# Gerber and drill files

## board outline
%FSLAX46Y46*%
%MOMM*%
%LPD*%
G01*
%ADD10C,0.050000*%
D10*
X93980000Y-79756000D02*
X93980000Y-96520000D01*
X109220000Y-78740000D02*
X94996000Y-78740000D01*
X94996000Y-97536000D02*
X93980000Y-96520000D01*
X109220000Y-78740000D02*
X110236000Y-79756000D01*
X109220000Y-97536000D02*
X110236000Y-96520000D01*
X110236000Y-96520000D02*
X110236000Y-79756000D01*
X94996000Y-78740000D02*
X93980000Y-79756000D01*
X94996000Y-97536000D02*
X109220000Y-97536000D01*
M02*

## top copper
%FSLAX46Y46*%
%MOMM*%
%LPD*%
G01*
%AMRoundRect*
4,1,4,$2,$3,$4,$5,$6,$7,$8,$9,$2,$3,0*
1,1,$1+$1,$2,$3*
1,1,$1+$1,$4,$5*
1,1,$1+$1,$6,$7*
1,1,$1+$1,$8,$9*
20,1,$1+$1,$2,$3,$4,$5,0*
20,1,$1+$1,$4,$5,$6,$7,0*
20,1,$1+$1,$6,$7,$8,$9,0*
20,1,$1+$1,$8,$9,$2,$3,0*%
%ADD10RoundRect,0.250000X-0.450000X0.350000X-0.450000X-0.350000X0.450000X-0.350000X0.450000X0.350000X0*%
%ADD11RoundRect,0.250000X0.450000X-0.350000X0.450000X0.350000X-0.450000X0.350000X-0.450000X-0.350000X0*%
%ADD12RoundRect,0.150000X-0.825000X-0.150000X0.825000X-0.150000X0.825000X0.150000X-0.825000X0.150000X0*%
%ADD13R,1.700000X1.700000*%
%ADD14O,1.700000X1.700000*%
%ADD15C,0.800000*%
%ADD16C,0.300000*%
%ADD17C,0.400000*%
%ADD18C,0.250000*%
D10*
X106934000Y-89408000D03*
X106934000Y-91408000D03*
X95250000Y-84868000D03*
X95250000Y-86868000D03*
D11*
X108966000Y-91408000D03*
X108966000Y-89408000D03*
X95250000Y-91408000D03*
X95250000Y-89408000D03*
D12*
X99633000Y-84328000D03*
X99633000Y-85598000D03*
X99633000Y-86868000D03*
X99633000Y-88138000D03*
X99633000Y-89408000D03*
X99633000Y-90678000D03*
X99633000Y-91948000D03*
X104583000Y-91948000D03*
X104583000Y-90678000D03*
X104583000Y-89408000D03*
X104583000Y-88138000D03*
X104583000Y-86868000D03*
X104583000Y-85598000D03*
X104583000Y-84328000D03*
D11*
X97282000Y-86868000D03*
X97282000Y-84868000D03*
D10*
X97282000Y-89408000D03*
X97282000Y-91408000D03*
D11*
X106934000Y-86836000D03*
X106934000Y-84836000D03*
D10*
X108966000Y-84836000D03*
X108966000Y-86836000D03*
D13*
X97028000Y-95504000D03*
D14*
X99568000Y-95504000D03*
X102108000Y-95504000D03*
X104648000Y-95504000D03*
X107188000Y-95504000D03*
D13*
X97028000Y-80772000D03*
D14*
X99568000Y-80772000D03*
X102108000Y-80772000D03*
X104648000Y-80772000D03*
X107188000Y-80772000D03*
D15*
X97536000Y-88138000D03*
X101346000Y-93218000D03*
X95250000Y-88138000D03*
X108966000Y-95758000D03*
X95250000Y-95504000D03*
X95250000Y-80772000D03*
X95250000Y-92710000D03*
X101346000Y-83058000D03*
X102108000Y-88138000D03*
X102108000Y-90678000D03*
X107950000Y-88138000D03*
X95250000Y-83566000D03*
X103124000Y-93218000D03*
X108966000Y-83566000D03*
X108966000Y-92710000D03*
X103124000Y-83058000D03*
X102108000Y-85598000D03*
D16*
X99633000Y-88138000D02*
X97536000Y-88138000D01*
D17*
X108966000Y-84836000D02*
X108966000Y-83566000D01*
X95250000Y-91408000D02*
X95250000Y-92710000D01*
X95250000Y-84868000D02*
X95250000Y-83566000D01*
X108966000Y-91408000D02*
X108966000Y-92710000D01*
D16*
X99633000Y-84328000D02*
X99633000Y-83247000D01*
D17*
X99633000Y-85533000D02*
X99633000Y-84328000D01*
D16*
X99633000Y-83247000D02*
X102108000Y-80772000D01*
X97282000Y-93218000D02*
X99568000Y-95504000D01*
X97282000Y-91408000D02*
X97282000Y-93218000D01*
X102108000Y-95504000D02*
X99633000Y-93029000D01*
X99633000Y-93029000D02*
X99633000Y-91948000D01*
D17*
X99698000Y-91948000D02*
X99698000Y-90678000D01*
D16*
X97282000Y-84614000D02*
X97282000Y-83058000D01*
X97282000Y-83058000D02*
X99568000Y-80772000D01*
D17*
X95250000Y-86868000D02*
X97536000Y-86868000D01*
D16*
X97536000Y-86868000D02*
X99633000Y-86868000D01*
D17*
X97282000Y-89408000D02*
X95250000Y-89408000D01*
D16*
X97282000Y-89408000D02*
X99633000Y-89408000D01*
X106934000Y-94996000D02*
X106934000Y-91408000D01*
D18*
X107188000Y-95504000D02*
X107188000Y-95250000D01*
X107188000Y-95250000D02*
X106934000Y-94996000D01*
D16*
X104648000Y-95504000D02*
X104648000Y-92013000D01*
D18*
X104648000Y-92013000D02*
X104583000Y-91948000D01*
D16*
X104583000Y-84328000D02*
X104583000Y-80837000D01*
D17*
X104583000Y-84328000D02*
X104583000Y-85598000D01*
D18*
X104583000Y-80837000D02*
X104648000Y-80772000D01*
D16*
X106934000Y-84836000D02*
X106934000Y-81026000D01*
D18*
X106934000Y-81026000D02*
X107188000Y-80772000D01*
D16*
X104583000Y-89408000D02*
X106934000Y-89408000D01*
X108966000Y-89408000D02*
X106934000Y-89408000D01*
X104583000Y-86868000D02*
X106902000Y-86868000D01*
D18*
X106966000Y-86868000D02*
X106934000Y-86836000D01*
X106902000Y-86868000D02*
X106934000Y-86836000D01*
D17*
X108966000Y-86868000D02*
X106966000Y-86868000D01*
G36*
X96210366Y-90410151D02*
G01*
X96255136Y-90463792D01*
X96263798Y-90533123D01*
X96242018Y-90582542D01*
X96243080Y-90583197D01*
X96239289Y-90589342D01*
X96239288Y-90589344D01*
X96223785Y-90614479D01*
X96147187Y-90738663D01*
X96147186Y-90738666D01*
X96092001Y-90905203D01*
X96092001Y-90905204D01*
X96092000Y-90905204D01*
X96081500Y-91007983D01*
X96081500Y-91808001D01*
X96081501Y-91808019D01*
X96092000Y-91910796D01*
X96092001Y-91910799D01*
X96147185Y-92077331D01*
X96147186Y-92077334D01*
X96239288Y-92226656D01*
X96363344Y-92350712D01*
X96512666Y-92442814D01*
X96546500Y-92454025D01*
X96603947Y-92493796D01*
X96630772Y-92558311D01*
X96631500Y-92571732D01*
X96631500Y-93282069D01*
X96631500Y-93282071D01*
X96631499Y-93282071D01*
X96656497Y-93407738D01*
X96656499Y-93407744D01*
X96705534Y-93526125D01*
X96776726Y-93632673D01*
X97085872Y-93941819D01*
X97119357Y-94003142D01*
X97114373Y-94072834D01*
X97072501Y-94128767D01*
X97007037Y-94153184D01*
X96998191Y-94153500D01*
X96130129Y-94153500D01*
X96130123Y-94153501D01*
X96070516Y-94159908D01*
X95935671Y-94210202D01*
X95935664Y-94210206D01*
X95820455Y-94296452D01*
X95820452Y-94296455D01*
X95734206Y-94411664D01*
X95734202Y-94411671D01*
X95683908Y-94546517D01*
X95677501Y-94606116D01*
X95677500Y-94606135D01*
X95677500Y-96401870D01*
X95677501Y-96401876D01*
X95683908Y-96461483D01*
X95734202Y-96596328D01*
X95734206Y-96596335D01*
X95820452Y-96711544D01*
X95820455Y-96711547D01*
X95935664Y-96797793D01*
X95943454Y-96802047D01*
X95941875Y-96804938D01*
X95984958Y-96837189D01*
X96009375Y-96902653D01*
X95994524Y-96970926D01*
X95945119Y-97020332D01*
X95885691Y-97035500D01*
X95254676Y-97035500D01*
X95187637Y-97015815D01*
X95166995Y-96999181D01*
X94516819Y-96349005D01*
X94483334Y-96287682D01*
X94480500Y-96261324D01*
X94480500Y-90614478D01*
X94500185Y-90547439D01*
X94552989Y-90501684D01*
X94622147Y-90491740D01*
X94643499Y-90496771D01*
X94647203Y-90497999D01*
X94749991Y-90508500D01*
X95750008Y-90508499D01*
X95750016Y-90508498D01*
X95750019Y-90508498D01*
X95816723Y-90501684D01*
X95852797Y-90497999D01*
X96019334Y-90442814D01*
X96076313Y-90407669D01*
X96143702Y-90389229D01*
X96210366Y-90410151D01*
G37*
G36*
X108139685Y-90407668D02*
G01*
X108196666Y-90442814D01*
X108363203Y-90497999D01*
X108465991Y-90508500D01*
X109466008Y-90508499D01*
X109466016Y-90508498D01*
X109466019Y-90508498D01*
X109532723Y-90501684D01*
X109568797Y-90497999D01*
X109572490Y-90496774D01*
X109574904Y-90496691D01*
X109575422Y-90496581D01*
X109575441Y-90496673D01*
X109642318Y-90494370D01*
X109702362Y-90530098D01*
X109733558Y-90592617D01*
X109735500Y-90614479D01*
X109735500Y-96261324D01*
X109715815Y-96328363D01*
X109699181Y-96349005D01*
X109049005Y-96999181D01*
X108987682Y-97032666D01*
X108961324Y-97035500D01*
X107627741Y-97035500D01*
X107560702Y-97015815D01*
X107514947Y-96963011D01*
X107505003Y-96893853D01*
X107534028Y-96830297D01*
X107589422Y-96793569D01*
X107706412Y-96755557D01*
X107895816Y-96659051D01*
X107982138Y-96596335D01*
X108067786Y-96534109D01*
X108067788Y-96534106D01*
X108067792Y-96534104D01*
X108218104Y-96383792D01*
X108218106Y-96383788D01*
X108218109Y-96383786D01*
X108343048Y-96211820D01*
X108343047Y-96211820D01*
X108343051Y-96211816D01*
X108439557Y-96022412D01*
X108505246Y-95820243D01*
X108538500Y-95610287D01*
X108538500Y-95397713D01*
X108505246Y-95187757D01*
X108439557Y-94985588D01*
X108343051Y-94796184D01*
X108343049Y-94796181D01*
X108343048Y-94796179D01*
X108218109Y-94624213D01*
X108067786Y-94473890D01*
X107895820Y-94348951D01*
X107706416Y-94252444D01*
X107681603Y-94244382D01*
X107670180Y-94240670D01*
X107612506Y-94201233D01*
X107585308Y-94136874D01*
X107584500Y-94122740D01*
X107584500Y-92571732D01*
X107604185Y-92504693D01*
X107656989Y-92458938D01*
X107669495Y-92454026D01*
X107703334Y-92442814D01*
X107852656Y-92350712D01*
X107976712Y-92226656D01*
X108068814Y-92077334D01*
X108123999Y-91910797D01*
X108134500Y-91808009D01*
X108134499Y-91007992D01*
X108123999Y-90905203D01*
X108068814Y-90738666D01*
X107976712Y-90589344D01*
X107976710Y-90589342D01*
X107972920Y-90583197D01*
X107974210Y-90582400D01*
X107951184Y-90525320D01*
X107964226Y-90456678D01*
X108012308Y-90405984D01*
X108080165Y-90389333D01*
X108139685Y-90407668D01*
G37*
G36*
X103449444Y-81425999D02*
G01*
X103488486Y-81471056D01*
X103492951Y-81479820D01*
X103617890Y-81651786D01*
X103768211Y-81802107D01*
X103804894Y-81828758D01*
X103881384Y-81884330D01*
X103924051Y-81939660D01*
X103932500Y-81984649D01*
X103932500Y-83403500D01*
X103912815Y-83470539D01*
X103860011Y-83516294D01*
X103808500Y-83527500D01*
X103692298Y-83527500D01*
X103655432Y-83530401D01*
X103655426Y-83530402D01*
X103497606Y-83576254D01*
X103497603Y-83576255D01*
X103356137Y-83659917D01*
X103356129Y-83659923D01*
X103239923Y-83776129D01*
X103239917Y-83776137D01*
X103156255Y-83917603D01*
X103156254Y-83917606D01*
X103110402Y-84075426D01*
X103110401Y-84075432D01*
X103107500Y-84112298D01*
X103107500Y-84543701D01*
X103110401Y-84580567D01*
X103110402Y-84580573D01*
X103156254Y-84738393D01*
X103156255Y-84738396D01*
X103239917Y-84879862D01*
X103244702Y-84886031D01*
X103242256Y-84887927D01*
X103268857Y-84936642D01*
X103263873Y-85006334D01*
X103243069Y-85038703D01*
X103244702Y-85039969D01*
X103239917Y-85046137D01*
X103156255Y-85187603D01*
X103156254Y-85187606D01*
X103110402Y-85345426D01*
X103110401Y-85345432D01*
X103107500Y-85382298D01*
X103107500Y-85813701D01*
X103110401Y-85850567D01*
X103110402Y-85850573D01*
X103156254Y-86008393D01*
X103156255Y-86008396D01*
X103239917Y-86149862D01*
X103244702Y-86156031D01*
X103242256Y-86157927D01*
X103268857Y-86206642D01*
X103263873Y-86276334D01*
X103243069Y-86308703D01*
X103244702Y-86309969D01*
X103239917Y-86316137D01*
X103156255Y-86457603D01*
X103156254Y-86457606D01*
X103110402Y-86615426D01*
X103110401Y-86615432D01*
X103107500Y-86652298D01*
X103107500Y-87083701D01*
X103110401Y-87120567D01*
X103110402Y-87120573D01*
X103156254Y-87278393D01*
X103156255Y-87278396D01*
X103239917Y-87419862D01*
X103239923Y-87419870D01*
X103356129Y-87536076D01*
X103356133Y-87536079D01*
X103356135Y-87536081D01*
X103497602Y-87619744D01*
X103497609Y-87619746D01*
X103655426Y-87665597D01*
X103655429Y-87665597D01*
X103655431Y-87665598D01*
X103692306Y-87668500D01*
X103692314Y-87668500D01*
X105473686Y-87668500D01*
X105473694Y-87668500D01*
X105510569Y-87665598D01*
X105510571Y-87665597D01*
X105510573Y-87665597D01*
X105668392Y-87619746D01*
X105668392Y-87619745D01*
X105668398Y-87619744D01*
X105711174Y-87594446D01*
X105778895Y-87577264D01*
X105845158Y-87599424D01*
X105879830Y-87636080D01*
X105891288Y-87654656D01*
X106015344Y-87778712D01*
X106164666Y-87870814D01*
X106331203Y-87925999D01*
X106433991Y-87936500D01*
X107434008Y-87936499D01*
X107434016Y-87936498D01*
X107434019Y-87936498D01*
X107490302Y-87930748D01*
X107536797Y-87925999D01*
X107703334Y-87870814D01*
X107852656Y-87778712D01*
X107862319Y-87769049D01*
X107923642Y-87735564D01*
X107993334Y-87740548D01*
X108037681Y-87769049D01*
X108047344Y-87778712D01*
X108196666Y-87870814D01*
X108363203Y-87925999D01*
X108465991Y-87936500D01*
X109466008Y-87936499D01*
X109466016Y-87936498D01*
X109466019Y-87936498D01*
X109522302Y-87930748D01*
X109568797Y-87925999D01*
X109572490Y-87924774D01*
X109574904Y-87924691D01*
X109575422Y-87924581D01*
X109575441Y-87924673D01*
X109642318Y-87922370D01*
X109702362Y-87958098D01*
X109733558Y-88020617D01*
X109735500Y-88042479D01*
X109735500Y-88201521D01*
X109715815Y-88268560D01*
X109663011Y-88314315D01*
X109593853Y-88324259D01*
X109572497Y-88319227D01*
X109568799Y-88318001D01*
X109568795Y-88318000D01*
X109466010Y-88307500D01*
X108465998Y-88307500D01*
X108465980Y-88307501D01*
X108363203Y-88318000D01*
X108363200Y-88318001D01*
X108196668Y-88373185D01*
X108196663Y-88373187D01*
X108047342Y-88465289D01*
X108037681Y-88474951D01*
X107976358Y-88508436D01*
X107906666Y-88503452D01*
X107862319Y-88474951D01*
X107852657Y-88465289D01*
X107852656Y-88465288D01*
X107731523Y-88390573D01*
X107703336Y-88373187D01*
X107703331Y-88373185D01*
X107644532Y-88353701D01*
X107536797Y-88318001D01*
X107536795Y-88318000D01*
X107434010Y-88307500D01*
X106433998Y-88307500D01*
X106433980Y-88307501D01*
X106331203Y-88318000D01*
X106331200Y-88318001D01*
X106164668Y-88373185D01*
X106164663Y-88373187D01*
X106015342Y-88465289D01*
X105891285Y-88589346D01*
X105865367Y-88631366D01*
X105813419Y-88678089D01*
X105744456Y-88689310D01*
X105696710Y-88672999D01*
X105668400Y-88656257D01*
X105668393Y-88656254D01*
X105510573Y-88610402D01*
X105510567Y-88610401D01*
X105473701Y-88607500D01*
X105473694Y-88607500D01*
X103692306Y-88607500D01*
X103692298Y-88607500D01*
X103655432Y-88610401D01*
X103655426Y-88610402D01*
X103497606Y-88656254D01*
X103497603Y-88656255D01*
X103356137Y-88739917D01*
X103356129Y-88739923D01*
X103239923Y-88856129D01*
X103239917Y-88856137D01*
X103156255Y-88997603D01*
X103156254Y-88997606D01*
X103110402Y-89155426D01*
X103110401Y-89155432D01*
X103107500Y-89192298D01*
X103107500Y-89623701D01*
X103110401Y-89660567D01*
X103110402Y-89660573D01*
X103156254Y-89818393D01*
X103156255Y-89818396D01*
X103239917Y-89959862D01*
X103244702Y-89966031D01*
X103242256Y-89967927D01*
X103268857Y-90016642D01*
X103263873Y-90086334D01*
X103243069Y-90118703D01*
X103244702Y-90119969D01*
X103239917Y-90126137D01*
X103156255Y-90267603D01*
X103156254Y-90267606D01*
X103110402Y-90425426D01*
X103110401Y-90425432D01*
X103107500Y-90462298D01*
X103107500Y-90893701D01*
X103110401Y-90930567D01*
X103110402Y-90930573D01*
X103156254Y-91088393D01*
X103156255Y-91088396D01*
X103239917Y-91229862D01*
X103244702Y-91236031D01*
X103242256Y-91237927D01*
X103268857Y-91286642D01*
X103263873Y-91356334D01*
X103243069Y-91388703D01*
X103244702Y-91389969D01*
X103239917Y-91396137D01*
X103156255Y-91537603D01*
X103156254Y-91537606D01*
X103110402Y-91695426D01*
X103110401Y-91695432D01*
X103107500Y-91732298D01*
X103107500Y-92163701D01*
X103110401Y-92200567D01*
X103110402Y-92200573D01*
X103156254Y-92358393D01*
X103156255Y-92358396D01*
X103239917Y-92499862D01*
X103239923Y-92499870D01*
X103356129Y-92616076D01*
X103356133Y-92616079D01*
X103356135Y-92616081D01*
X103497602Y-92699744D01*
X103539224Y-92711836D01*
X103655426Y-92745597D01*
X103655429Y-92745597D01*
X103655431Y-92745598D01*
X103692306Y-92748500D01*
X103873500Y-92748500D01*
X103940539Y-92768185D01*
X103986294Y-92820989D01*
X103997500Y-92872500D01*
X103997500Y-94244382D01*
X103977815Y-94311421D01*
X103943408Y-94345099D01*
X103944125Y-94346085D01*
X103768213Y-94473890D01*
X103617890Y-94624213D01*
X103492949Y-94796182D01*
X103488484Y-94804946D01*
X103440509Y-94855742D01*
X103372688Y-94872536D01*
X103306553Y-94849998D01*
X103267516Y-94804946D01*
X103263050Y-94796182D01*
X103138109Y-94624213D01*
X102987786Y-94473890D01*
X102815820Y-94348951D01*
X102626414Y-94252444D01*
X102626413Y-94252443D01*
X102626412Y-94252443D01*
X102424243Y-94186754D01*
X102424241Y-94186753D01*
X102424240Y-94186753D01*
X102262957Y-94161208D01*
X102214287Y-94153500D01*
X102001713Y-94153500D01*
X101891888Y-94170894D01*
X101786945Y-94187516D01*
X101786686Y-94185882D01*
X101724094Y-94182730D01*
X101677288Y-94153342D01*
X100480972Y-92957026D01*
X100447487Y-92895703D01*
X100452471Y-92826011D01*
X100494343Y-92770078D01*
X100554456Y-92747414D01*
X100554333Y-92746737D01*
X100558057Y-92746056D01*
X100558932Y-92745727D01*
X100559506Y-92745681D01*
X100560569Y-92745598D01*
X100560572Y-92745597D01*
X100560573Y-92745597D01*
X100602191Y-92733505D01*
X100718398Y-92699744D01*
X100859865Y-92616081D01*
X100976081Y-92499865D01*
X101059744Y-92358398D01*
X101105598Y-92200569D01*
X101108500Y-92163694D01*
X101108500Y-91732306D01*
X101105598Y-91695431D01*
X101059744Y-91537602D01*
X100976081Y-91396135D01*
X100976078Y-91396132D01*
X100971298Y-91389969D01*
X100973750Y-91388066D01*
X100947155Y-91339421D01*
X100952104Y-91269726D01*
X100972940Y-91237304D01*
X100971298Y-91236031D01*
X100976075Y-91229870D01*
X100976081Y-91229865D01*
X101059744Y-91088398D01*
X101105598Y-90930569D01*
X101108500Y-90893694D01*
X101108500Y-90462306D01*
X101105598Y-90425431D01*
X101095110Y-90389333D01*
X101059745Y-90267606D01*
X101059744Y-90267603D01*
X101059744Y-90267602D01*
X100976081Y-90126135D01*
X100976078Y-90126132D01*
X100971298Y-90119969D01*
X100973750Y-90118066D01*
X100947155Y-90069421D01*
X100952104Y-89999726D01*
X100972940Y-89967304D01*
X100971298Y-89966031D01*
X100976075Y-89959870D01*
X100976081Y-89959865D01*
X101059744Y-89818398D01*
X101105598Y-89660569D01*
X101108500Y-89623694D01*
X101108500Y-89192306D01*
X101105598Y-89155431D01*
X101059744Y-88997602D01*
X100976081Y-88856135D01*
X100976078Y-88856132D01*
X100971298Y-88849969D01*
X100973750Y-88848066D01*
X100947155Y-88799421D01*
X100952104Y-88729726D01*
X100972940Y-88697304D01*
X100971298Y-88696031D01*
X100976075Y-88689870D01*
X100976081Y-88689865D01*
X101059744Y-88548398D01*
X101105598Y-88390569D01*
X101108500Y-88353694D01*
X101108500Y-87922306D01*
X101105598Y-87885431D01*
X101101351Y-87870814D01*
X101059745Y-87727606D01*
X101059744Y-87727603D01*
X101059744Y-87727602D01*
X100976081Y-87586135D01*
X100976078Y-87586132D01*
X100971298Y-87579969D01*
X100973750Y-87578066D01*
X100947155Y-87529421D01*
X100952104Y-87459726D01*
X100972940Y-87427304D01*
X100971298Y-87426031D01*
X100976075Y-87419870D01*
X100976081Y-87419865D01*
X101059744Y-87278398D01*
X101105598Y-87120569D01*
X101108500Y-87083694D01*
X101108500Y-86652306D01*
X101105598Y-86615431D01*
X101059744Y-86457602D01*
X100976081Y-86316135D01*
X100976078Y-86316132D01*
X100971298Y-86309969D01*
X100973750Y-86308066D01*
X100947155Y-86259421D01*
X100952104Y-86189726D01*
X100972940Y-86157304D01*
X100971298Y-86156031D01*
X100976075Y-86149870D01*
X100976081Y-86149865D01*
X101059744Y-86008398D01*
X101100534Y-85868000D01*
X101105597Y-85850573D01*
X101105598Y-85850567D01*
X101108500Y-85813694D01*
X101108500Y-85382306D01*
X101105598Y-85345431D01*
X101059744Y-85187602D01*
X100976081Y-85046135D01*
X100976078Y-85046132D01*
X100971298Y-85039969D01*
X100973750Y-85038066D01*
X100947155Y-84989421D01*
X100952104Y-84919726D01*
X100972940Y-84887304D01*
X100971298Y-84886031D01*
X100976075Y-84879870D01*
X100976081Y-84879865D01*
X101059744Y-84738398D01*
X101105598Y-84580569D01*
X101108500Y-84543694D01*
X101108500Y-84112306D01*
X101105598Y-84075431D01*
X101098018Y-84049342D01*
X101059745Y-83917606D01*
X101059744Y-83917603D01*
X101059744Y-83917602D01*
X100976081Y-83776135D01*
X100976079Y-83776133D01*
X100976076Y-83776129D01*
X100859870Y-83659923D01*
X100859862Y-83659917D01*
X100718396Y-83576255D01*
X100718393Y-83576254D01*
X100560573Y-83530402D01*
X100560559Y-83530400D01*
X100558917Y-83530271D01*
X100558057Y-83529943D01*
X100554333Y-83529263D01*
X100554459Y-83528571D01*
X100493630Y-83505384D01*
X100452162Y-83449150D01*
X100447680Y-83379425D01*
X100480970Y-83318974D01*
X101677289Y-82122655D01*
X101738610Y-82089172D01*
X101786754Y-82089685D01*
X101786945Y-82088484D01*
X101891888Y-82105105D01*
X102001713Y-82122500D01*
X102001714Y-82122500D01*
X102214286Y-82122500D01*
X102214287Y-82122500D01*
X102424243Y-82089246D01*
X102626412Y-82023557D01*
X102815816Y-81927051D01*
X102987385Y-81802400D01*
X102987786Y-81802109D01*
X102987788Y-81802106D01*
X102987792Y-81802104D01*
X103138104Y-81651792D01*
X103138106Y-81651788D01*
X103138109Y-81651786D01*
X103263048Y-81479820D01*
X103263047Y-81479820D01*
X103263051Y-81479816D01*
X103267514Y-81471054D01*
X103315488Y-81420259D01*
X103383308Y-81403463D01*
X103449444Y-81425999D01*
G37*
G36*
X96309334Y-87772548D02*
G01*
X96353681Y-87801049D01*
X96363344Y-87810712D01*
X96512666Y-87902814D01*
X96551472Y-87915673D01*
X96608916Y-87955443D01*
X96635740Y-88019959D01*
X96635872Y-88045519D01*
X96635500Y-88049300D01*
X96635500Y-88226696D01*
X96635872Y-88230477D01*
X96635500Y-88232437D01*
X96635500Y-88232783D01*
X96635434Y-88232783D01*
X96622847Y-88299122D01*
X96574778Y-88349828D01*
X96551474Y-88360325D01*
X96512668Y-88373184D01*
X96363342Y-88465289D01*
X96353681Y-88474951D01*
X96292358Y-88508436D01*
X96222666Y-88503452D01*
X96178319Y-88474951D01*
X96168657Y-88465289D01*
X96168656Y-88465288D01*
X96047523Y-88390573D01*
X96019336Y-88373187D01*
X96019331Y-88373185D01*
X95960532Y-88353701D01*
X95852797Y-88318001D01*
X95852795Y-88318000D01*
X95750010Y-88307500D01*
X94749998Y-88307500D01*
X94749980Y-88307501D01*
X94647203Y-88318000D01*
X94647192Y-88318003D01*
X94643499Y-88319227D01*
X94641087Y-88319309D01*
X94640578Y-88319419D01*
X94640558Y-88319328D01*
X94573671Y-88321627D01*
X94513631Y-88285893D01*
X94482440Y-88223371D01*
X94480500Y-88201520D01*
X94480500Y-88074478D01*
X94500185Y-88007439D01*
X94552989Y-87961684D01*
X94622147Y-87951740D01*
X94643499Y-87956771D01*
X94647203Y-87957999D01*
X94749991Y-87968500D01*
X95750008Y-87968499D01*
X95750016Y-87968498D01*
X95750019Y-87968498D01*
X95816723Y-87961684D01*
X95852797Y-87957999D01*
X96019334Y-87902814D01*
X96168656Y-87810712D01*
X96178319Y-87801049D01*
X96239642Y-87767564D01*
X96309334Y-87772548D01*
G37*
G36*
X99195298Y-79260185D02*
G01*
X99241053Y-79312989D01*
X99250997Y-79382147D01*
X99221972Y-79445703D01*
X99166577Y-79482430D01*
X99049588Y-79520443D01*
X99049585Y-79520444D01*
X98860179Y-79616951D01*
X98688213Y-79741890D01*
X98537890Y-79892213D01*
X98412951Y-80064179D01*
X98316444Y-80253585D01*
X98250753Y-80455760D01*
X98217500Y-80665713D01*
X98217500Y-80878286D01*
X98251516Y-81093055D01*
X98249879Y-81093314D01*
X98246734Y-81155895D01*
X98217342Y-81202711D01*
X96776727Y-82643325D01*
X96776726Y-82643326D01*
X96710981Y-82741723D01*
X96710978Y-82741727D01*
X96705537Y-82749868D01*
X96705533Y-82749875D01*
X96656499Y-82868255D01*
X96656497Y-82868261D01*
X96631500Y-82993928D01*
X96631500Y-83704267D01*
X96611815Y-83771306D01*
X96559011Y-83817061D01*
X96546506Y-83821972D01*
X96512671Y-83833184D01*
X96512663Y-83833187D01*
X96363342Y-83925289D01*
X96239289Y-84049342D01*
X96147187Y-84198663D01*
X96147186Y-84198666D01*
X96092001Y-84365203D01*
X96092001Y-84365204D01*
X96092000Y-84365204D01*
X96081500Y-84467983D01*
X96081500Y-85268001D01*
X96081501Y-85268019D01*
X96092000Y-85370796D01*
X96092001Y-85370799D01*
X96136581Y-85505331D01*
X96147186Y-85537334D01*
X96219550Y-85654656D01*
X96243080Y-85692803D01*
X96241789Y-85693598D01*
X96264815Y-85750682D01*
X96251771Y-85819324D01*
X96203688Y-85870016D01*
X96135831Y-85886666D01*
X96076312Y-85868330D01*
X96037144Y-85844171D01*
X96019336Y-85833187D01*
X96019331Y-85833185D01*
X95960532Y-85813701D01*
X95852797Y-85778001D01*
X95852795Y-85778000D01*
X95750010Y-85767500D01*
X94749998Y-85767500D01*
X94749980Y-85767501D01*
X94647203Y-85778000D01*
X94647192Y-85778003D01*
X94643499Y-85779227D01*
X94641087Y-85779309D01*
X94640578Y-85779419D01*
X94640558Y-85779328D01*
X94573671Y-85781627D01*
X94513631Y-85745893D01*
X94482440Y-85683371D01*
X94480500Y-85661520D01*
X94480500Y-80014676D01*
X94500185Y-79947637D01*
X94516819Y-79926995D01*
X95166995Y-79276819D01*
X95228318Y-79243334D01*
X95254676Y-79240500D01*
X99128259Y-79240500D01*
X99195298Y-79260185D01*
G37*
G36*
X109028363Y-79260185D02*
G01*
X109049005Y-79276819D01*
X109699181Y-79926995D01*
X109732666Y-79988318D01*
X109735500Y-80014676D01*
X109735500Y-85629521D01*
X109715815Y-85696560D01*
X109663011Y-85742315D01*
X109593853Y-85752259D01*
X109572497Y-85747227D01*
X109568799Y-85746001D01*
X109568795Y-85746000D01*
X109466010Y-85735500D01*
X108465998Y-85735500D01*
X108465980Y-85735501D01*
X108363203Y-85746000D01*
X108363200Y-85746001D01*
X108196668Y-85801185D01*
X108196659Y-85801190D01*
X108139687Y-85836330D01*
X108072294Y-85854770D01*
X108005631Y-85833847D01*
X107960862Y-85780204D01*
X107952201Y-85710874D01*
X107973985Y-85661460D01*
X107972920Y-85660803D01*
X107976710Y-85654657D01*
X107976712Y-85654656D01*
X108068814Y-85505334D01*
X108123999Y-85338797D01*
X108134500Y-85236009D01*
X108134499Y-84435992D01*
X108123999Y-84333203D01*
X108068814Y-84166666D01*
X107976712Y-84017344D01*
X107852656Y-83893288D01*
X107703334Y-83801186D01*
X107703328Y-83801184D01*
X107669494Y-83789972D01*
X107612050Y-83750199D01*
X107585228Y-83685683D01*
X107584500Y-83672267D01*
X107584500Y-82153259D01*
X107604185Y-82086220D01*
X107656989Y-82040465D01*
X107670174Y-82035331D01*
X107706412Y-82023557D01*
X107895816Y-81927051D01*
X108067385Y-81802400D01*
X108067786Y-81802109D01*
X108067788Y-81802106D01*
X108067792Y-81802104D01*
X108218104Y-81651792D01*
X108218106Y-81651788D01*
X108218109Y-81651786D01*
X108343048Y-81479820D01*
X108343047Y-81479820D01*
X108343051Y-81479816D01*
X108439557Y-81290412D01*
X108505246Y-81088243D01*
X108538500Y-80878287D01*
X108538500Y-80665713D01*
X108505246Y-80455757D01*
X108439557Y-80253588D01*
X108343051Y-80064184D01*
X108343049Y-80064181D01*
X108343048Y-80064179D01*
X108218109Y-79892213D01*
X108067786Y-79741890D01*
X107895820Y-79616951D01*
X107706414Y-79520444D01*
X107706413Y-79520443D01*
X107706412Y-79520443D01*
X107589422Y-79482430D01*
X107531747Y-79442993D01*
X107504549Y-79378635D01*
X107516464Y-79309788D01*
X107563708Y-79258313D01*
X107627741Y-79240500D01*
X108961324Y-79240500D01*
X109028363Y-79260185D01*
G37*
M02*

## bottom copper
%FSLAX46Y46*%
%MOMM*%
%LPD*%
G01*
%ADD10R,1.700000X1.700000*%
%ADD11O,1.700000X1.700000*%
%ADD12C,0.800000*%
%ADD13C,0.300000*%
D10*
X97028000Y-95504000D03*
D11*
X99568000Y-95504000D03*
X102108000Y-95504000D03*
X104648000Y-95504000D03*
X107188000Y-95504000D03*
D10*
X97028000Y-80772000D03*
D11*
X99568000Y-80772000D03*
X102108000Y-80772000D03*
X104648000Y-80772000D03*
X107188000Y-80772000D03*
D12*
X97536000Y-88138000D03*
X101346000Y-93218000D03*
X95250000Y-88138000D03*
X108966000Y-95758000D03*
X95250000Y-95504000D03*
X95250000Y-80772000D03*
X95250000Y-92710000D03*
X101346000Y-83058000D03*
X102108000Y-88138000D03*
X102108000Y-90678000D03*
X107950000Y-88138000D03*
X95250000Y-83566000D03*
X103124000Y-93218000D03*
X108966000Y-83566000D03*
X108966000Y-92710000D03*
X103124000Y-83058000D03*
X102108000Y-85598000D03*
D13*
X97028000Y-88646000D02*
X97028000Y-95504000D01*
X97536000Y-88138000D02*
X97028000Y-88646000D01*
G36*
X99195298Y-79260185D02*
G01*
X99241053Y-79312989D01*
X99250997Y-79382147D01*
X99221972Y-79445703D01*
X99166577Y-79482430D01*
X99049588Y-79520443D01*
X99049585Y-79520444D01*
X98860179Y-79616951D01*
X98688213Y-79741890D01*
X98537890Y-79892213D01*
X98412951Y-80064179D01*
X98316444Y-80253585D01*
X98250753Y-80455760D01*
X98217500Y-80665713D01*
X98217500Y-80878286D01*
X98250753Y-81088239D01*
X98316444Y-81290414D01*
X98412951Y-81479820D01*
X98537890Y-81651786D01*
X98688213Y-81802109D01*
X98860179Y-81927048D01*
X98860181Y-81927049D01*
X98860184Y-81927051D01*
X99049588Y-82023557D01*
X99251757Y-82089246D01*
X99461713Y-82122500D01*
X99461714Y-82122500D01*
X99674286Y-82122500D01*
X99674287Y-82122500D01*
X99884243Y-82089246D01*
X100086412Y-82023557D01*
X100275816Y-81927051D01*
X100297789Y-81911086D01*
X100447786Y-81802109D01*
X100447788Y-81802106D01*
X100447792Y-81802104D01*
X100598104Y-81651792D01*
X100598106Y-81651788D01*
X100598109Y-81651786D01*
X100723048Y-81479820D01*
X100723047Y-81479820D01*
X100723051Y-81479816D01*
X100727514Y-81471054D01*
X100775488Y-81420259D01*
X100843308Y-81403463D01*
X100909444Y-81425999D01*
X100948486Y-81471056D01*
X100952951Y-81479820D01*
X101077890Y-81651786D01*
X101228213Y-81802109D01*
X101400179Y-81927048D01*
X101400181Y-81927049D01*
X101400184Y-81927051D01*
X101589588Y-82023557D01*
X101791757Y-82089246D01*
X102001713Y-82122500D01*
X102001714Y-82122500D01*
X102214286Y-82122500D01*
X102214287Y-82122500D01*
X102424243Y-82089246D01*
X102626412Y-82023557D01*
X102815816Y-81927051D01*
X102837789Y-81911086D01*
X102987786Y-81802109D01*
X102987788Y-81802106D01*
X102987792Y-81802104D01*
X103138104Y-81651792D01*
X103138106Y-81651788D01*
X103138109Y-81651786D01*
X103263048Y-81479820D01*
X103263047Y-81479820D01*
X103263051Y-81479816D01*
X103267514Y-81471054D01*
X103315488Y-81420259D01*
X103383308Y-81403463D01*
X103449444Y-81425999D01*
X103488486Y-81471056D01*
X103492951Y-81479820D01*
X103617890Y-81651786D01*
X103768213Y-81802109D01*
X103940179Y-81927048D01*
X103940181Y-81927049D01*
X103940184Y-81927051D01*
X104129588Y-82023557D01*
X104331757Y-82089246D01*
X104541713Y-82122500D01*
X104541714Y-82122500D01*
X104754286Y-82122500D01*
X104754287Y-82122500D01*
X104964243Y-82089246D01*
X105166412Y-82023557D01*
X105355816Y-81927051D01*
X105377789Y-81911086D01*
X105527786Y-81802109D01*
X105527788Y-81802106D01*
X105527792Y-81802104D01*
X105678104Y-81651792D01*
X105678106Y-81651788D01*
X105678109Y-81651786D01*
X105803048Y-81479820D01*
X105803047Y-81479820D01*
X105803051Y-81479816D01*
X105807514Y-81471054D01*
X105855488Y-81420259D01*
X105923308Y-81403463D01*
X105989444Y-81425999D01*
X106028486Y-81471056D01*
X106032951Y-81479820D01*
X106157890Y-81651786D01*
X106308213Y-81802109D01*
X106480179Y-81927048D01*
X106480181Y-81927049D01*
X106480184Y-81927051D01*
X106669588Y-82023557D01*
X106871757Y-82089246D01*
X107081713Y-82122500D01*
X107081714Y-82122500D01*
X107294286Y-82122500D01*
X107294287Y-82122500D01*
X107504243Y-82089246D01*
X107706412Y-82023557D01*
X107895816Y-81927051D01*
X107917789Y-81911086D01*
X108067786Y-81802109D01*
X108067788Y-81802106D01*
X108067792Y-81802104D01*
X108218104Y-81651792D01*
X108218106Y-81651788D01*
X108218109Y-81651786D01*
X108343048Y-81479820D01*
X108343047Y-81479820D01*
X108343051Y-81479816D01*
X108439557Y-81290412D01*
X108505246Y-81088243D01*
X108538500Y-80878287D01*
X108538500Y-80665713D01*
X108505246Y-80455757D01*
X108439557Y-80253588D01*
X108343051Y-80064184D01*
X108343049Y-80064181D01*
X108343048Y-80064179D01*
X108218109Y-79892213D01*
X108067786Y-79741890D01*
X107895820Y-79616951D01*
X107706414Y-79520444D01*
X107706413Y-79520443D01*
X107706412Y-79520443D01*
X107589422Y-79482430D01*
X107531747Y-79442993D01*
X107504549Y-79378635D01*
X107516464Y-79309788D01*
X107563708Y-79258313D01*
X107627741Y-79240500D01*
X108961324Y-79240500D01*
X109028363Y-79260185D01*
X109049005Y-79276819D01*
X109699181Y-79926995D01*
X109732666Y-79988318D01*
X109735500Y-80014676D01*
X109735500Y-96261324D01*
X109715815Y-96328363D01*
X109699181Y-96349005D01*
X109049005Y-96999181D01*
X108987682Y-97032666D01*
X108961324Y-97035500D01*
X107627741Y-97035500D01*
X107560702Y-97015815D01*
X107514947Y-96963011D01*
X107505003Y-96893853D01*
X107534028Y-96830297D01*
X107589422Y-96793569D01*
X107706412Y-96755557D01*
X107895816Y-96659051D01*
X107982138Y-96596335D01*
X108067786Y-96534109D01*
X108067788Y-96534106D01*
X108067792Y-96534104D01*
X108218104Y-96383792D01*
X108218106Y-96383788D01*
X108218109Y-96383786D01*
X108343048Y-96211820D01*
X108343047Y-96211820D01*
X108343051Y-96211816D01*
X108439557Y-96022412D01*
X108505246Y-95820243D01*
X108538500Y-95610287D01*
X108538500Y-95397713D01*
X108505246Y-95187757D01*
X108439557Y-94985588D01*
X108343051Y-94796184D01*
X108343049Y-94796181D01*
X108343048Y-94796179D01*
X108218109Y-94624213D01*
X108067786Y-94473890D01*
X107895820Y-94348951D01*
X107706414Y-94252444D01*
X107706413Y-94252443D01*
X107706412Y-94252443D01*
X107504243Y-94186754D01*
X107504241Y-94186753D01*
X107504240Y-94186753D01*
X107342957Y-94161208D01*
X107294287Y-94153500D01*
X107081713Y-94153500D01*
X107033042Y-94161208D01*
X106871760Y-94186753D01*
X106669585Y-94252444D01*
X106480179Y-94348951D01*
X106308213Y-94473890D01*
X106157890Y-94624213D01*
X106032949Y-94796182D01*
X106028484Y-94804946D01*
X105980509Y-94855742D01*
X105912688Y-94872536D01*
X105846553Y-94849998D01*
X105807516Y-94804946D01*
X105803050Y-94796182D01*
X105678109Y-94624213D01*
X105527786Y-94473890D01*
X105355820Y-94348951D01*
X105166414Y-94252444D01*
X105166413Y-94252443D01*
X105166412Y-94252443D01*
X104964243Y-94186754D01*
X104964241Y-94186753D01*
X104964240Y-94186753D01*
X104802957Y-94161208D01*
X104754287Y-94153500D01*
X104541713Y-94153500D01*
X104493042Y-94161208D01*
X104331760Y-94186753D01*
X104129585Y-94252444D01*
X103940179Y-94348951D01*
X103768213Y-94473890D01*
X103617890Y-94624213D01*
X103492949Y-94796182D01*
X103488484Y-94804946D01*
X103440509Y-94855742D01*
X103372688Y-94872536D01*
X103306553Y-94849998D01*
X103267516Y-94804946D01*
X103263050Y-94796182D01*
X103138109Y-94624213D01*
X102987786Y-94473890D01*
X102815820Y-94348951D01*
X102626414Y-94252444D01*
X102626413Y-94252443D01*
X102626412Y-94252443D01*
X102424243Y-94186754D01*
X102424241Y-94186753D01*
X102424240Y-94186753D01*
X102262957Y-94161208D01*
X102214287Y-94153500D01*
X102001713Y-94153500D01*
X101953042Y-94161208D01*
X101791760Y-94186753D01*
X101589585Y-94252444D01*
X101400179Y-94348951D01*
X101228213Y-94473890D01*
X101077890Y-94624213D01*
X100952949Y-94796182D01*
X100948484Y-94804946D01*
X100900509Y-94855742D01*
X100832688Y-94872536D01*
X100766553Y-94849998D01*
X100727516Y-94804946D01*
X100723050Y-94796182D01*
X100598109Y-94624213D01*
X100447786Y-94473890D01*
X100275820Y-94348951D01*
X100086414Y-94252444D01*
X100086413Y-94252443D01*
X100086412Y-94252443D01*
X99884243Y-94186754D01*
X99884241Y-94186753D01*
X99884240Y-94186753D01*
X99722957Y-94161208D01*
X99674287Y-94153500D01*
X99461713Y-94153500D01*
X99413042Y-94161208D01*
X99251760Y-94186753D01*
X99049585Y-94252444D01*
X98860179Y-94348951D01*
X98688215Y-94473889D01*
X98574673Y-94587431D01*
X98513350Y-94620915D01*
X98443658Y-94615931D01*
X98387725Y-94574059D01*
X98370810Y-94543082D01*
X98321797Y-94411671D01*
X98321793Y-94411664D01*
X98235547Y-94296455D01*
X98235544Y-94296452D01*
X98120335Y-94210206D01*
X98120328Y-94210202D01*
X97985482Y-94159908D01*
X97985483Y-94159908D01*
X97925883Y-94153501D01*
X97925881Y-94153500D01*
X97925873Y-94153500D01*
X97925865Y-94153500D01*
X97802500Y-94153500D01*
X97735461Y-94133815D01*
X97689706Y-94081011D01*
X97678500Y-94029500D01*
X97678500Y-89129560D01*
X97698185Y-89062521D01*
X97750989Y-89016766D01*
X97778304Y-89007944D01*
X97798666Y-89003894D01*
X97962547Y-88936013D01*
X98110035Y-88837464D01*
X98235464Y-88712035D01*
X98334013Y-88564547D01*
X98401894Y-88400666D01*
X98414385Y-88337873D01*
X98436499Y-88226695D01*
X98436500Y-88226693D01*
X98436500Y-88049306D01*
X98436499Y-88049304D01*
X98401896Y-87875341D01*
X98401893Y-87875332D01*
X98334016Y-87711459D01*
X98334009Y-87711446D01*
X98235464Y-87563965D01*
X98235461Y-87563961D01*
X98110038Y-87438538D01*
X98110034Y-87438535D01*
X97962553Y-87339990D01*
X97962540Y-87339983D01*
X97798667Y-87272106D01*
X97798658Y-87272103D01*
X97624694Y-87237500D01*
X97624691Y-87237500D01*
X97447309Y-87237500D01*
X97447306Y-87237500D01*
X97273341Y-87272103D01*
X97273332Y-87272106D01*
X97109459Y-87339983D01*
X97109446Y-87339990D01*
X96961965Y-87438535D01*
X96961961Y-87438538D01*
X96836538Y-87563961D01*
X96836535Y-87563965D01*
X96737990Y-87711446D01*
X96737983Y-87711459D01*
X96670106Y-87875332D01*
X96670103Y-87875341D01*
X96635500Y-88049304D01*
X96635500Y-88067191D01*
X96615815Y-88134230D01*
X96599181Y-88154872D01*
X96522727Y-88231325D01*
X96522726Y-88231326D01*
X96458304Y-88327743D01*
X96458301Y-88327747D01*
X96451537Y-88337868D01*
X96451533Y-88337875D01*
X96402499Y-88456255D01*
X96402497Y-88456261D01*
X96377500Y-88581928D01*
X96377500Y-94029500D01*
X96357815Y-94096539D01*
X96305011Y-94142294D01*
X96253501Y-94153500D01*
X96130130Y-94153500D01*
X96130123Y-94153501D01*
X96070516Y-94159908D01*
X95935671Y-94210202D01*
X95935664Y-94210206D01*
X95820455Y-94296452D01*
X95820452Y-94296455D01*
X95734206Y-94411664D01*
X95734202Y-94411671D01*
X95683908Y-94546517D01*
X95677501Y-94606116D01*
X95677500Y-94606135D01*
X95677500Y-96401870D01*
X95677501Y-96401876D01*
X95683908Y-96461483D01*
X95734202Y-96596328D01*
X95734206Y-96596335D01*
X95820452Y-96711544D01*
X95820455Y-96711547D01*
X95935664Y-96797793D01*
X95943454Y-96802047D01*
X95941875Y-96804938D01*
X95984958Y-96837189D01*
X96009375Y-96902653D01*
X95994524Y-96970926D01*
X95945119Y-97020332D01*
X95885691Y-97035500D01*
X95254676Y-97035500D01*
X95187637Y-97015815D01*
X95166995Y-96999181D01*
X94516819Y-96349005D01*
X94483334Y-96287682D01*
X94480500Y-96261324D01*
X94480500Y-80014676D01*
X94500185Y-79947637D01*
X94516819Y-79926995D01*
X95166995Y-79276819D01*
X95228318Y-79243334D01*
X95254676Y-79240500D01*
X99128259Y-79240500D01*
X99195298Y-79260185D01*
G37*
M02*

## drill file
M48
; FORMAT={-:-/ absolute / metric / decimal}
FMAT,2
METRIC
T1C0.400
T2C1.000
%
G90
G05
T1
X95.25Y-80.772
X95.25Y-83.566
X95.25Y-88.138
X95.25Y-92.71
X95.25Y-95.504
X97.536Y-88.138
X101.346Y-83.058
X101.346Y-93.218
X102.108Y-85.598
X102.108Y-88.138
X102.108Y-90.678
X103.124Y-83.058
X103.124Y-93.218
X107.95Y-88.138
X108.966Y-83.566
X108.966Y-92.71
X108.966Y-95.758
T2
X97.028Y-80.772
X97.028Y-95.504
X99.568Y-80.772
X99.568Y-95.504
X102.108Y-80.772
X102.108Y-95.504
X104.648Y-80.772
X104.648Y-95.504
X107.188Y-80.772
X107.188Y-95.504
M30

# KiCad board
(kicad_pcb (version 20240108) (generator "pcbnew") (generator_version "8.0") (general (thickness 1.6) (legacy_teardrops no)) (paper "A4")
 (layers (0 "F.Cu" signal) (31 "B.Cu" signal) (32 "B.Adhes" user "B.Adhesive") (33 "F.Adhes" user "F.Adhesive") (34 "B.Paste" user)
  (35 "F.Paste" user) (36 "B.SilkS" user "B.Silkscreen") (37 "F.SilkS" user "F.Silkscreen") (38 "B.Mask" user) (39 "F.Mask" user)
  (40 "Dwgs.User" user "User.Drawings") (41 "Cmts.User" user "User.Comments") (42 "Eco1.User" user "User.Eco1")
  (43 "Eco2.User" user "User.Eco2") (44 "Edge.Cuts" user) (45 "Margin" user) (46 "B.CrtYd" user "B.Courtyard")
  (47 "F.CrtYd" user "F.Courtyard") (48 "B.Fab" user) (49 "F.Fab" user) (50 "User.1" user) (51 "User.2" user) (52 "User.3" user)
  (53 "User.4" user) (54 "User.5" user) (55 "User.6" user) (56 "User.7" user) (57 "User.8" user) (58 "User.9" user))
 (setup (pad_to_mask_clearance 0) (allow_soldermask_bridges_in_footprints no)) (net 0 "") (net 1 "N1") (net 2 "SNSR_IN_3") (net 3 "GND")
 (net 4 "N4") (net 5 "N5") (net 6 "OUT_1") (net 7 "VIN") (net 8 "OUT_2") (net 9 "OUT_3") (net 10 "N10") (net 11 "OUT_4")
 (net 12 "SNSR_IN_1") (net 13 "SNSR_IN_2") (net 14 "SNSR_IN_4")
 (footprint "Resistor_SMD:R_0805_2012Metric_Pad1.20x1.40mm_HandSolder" (layer "F.Cu") (at 106.934 90.408 -90)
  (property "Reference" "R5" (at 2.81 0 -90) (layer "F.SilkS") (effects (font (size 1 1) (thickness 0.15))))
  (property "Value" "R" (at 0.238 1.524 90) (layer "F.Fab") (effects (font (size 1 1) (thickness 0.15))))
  (pad "1" smd roundrect (at -1 0 270) (size 1.2 1.4) (layers "F.Cu" "F.Paste" "F.Mask") (roundrect_rratio 0.208333) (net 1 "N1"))
  (pad "2" smd roundrect (at 1 0 270) (size 1.2 1.4) (layers "F.Cu" "F.Paste" "F.Mask") (roundrect_rratio 0.208333) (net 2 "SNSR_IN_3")))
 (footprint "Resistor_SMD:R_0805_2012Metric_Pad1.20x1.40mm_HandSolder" (layer "F.Cu") (at 95.25 85.868 -90)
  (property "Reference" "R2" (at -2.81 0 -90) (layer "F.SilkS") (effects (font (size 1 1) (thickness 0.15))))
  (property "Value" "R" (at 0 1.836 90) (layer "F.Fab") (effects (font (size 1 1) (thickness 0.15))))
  (pad "1" smd roundrect (at -1 0 270) (size 1.2 1.4) (layers "F.Cu" "F.Paste" "F.Mask") (roundrect_rratio 0.208333) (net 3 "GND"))
  (pad "2" smd roundrect (at 1 0 270) (size 1.2 1.4) (layers "F.Cu" "F.Paste" "F.Mask") (roundrect_rratio 0.208333) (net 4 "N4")))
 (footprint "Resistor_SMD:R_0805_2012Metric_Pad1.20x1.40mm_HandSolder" (layer "F.Cu") (at 108.966 90.408 90)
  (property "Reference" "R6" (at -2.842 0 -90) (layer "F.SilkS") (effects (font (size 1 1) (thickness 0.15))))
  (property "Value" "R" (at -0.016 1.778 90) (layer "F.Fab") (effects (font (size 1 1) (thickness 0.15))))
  (pad "1" smd roundrect (at -1 0 90) (size 1.2 1.4) (layers "F.Cu" "F.Paste" "F.Mask") (roundrect_rratio 0.208333) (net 3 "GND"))
  (pad "2" smd roundrect (at 1 0 90) (size 1.2 1.4) (layers "F.Cu" "F.Paste" "F.Mask") (roundrect_rratio 0.208333) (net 1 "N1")))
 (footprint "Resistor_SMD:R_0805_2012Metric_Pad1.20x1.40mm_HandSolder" (layer "F.Cu") (at 95.25 90.408 90)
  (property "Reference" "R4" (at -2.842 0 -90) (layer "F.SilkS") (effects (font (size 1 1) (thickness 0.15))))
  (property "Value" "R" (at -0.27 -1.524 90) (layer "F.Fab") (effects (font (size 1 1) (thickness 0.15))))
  (pad "1" smd roundrect (at -1 0 90) (size 1.2 1.4) (layers "F.Cu" "F.Paste" "F.Mask") (roundrect_rratio 0.208333) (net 3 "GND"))
  (pad "2" smd roundrect (at 1 0 90) (size 1.2 1.4) (layers "F.Cu" "F.Paste" "F.Mask") (roundrect_rratio 0.208333) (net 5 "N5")))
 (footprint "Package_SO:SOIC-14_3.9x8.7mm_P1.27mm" (layer "F.Cu") (at 102.108 88.138)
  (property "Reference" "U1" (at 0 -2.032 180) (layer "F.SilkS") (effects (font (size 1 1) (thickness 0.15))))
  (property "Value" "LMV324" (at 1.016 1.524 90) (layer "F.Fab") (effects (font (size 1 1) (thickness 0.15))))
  (pad "1" smd roundrect (at -2.475 -3.81) (size 1.95 0.6) (layers "F.Cu" "F.Paste" "F.Mask") (roundrect_rratio 0.25) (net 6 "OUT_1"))
  (pad "2" smd roundrect (at -2.475 -2.54) (size 1.95 0.6) (layers "F.Cu" "F.Paste" "F.Mask") (roundrect_rratio 0.25) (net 6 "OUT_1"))
  (pad "3" smd roundrect (at -2.475 -1.27) (size 1.95 0.6) (layers "F.Cu" "F.Paste" "F.Mask") (roundrect_rratio 0.25) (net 4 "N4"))
  (pad "4" smd roundrect (at -2.475 0) (size 1.95 0.6) (layers "F.Cu" "F.Paste" "F.Mask") (roundrect_rratio 0.25) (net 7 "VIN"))
  (pad "5" smd roundrect (at -2.475 1.27) (size 1.95 0.6) (layers "F.Cu" "F.Paste" "F.Mask") (roundrect_rratio 0.25) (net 5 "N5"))
  (pad "6" smd roundrect (at -2.475 2.54) (size 1.95 0.6) (layers "F.Cu" "F.Paste" "F.Mask") (roundrect_rratio 0.25) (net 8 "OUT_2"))
  (pad "7" smd roundrect (at -2.475 3.81) (size 1.95 0.6) (layers "F.Cu" "F.Paste" "F.Mask") (roundrect_rratio 0.25) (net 8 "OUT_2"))
  (pad "8" smd roundrect (at 2.475 3.81) (size 1.95 0.6) (layers "F.Cu" "F.Paste" "F.Mask") (roundrect_rratio 0.25) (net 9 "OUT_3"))
  (pad "9" smd roundrect (at 2.475 2.54) (size 1.95 0.6) (layers "F.Cu" "F.Paste" "F.Mask") (roundrect_rratio 0.25) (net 9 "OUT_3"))
  (pad "10" smd roundrect (at 2.475 1.27) (size 1.95 0.6) (layers "F.Cu" "F.Paste" "F.Mask") (roundrect_rratio 0.25) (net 1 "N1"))
  (pad "11" smd roundrect (at 2.475 0) (size 1.95 0.6) (layers "F.Cu" "F.Paste" "F.Mask") (roundrect_rratio 0.25) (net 3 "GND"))
  (pad "12" smd roundrect (at 2.475 -1.27) (size 1.95 0.6) (layers "F.Cu" "F.Paste" "F.Mask") (roundrect_rratio 0.25) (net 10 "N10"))
  (pad "13" smd roundrect (at 2.475 -2.54) (size 1.95 0.6) (layers "F.Cu" "F.Paste" "F.Mask") (roundrect_rratio 0.25) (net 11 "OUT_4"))
  (pad "14" smd roundrect (at 2.475 -3.81) (size 1.95 0.6) (layers "F.Cu" "F.Paste" "F.Mask") (roundrect_rratio 0.25) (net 11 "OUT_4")))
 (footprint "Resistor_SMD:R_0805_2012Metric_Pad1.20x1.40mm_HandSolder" (layer "F.Cu") (at 97.282 85.868 90)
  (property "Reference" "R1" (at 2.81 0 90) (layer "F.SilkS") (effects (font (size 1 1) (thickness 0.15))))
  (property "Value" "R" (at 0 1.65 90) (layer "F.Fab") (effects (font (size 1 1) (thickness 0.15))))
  (pad "1" smd roundrect (at -1 0 90) (size 1.2 1.4) (layers "F.Cu" "F.Paste" "F.Mask") (roundrect_rratio 0.208333) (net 4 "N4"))
  (pad "2" smd roundrect (at 1 0 90) (size 1.2 1.4) (layers "F.Cu" "F.Paste" "F.Mask") (roundrect_rratio 0.208333) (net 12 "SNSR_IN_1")))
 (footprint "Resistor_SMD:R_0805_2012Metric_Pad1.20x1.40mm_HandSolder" (layer "F.Cu") (at 97.282 90.408 -90)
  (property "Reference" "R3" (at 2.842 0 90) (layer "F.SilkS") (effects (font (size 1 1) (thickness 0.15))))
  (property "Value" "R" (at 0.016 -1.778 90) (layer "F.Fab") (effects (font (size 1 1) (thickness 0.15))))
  (pad "1" smd roundrect (at -1 0 270) (size 1.2 1.4) (layers "F.Cu" "F.Paste" "F.Mask") (roundrect_rratio 0.208333) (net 5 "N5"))
  (pad "2" smd roundrect (at 1 0 270) (size 1.2 1.4) (layers "F.Cu" "F.Paste" "F.Mask") (roundrect_rratio 0.208333) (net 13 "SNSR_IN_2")))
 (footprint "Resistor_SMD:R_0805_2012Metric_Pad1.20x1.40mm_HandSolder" (layer "F.Cu") (at 106.934 85.836 90)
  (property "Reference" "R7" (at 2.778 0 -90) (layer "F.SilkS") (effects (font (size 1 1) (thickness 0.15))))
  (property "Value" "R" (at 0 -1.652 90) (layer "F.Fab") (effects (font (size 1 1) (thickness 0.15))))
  (pad "1" smd roundrect (at -1 0 90) (size 1.2 1.4) (layers "F.Cu" "F.Paste" "F.Mask") (roundrect_rratio 0.208333) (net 10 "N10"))
  (pad "2" smd roundrect (at 1 0 90) (size 1.2 1.4) (layers "F.Cu" "F.Paste" "F.Mask") (roundrect_rratio 0.208333) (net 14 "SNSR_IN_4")))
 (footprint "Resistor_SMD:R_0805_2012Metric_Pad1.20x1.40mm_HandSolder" (layer "F.Cu") (at 108.966 85.836 -90)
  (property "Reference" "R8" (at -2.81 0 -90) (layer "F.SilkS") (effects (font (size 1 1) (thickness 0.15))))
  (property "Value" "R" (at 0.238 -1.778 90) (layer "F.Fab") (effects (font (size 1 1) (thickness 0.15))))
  (pad "1" smd roundrect (at -1 0 270) (size 1.2 1.4) (layers "F.Cu" "F.Paste" "F.Mask") (roundrect_rratio 0.208333) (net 3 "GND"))
  (pad "2" smd roundrect (at 1 0 270) (size 1.2 1.4) (layers "F.Cu" "F.Paste" "F.Mask") (roundrect_rratio 0.208333) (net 10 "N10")))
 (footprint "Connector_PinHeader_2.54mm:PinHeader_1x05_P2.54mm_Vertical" (layer "B.Cu") (at 97.028 95.504 -90)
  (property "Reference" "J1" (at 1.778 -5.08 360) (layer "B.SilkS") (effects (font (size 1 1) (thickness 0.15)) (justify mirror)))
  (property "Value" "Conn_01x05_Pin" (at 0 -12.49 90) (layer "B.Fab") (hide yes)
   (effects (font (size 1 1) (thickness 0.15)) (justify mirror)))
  (pad "1" thru_hole rect (at 0 0 270) (size 1.7 1.7) (drill 1) (layers "*.Cu" "*.Mask") (remove_unused_layers no) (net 7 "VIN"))
  (pad "2" thru_hole oval (at 0 -2.54 270) (size 1.7 1.7) (drill 1) (layers "*.Cu" "*.Mask") (remove_unused_layers no) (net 13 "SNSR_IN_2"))
  (pad "3" thru_hole oval (at 0 -5.08 270) (size 1.7 1.7) (drill 1) (layers "*.Cu" "*.Mask") (remove_unused_layers no) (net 8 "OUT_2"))
  (pad "4" thru_hole oval (at 0 -7.62 270) (size 1.7 1.7) (drill 1) (layers "*.Cu" "*.Mask") (remove_unused_layers no) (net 9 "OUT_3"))
  (pad "5" thru_hole oval (at 0 -10.16 270) (size 1.7 1.7) (drill 1) (layers "*.Cu" "*.Mask") (remove_unused_layers no) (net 2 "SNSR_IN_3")))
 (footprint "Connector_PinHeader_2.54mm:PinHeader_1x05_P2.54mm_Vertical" (layer "B.Cu") (at 97.028 80.772 -90)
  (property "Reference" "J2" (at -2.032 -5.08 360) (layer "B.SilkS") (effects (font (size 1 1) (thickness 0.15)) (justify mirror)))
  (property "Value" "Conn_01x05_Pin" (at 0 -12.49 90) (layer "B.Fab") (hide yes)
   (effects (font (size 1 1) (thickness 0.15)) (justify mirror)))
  (pad "1" thru_hole rect (at 0 0 270) (size 1.7 1.7) (drill 1) (layers "*.Cu" "*.Mask") (remove_unused_layers no) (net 3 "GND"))
  (pad "2" thru_hole oval (at 0 -2.54 270) (size 1.7 1.7) (drill 1) (layers "*.Cu" "*.Mask") (remove_unused_layers no) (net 12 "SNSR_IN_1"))
  (pad "3" thru_hole oval (at 0 -5.08 270) (size 1.7 1.7) (drill 1) (layers "*.Cu" "*.Mask") (remove_unused_layers no) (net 6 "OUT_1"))
  (pad "4" thru_hole oval (at 0 -7.62 270) (size 1.7 1.7) (drill 1) (layers "*.Cu" "*.Mask") (remove_unused_layers no) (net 11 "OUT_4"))
  (pad "5" thru_hole oval (at 0 -10.16 270) (size 1.7 1.7) (drill 1) (layers "*.Cu" "*.Mask") (remove_unused_layers no) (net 14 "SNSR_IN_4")))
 (gr_line (start 93.98 79.756) (end 93.98 96.52) (stroke (width 0.05) (type default)) (layer "Edge.Cuts"))
 (gr_line (start 109.22 78.74) (end 94.996 78.74) (stroke (width 0.05) (type default)) (layer "Edge.Cuts"))
 (gr_line (start 94.996 97.536) (end 93.98 96.52) (stroke (width 0.05) (type default)) (layer "Edge.Cuts"))
 (gr_line (start 109.22 78.74) (end 110.236 79.756) (stroke (width 0.05) (type default)) (layer "Edge.Cuts"))
 (gr_line (start 109.22 97.536) (end 110.236 96.52) (stroke (width 0.05) (type default)) (layer "Edge.Cuts"))
 (gr_line (start 110.236 96.52) (end 110.236 79.756) (stroke (width 0.05) (type default)) (layer "Edge.Cuts"))
 (gr_line (start 94.996 78.74) (end 93.98 79.756) (stroke (width 0.05) (type default)) (layer "Edge.Cuts"))
 (gr_line (start 94.996 97.536) (end 109.22 97.536) (stroke (width 0.05) (type default)) (layer "Edge.Cuts"))
 (segment (start 99.633 88.138) (end 97.536 88.138) (width 0.3) (layer "F.Cu") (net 7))
 (via (at 97.536 88.138) (size 0.8) (drill 0.4) (layers "F.Cu" "B.Cu") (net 7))
 (segment (start 97.028 88.646) (end 97.028 95.504) (width 0.3) (layer "B.Cu") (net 7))
 (segment (start 97.536 88.138) (end 97.028 88.646) (width 0.3) (layer "B.Cu") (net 7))
 (segment (start 108.966 84.836) (end 108.966 83.566) (width 0.4) (layer "F.Cu") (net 3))
 (segment (start 95.25 91.408) (end 95.25 92.71) (width 0.4) (layer "F.Cu") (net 3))
 (segment (start 95.25 84.868) (end 95.25 83.566) (width 0.4) (layer "F.Cu") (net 3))
 (segment (start 108.966 91.408) (end 108.966 92.71) (width 0.4) (layer "F.Cu") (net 3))
 (via (at 101.346 93.218) (size 0.8) (drill 0.4) (layers "F.Cu" "B.Cu") (free yes) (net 3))
 (via (at 95.25 88.138) (size 0.8) (drill 0.4) (layers "F.Cu" "B.Cu") (free yes) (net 3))
 (via (at 108.966 95.758) (size 0.8) (drill 0.4) (layers "F.Cu" "B.Cu") (free yes) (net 3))
 (via (at 95.25 95.504) (size 0.8) (drill 0.4) (layers "F.Cu" "B.Cu") (free yes) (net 3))
 (via (at 95.25 80.772) (size 0.8) (drill 0.4) (layers "F.Cu" "B.Cu") (free yes) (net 3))
 (via (at 95.25 92.71) (size 0.8) (drill 0.4) (layers "F.Cu" "B.Cu") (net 3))
 (via (at 101.346 83.058) (size 0.8) (drill 0.4) (layers "F.Cu" "B.Cu") (free yes) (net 3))
 (via (at 102.108 88.138) (size 0.8) (drill 0.4) (layers "F.Cu" "B.Cu") (free yes) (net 3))
 (via (at 102.108 90.678) (size 0.8) (drill 0.4) (layers "F.Cu" "B.Cu") (free yes) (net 3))
 (via (at 107.95 88.138) (size 0.8) (drill 0.4) (layers "F.Cu" "B.Cu") (free yes) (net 3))
 (via (at 95.25 83.566) (size 0.8) (drill 0.4) (layers "F.Cu" "B.Cu") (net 3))
 (via (at 103.124 93.218) (size 0.8) (drill 0.4) (layers "F.Cu" "B.Cu") (free yes) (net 3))
 (via (at 108.966 83.566) (size 0.8) (drill 0.4) (layers "F.Cu" "B.Cu") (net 3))
 (via (at 108.966 92.71) (size 0.8) (drill 0.4) (layers "F.Cu" "B.Cu") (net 3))
 (via (at 103.124 83.058) (size 0.8) (drill 0.4) (layers "F.Cu" "B.Cu") (free yes) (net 3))
 (via (at 102.108 85.598) (size 0.8) (drill 0.4) (layers "F.Cu" "B.Cu") (free yes) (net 3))
 (segment (start 99.633 84.328) (end 99.633 83.247) (width 0.3) (layer "F.Cu") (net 6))
 (segment (start 99.633 85.533) (end 99.633 84.328) (width 0.4) (layer "F.Cu") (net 6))
 (segment (start 99.633 83.247) (end 102.108 80.772) (width 0.3) (layer "F.Cu") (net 6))
 (segment (start 97.282 93.218) (end 99.568 95.504) (width 0.3) (layer "F.Cu") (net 13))
 (segment (start 97.282 91.408) (end 97.282 93.218) (width 0.3) (layer "F.Cu") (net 13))
 (segment (start 102.108 95.504) (end 99.633 93.029) (width 0.3) (layer "F.Cu") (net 8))
 (segment (start 99.633 93.029) (end 99.633 91.948) (width 0.3) (layer "F.Cu") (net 8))
 (segment (start 99.698 91.948) (end 99.698 90.678) (width 0.4) (layer "F.Cu") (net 8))
 (segment (start 97.282 84.614) (end 97.282 83.058) (width 0.3) (layer "F.Cu") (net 12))
 (segment (start 97.282 83.058) (end 99.568 80.772) (width 0.3) (layer "F.Cu") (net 12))
 (segment (start 95.25 86.868) (end 97.536 86.868) (width 0.4) (layer "F.Cu") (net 4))
 (segment (start 97.536 86.868) (end 99.633 86.868) (width 0.3) (layer "F.Cu") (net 4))
 (segment (start 97.282 89.408) (end 95.25 89.408) (width 0.4) (layer "F.Cu") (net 5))
 (segment (start 97.282 89.408) (end 99.633 89.408) (width 0.3) (layer "F.Cu") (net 5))
 (segment (start 106.934 94.996) (end 106.934 91.408) (width 0.3) (layer "F.Cu") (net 2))
 (segment (start 107.188 95.504) (end 107.188 95.25) (width 0.25) (layer "F.Cu") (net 2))
 (segment (start 107.188 95.25) (end 106.934 94.996) (width 0.25) (layer "F.Cu") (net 2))
 (segment (start 104.648 95.504) (end 104.648 92.013) (width 0.3) (layer "F.Cu") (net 9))
 (segment (start 104.648 92.013) (end 104.583 91.948) (width 0.25) (layer "F.Cu") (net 9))
 (segment (start 104.583 84.328) (end 104.583 80.837) (width 0.3) (layer "F.Cu") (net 11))
 (segment (start 104.583 84.328) (end 104.583 85.598) (width 0.4) (layer "F.Cu") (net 11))
 (segment (start 104.583 80.837) (end 104.648 80.772) (width 0.25) (layer "F.Cu") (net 11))
 (segment (start 106.934 84.836) (end 106.934 81.026) (width 0.3) (layer "F.Cu") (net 14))
 (segment (start 106.934 81.026) (end 107.188 80.772) (width 0.25) (layer "F.Cu") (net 14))
 (segment (start 104.583 89.408) (end 106.934 89.408) (width 0.3) (layer "F.Cu") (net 1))
 (segment (start 108.966 89.408) (end 106.934 89.408) (width 0.3) (layer "F.Cu") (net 1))
 (segment (start 104.583 86.868) (end 106.902 86.868) (width 0.3) (layer "F.Cu") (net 10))
 (segment (start 106.966 86.868) (end 106.934 86.836) (width 0.25) (layer "F.Cu") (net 10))
 (segment (start 106.902 86.868) (end 106.934 86.836) (width 0.25) (layer "F.Cu") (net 10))
 (segment (start 108.966 86.868) (end 106.966 86.868) (width 0.4) (layer "F.Cu") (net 10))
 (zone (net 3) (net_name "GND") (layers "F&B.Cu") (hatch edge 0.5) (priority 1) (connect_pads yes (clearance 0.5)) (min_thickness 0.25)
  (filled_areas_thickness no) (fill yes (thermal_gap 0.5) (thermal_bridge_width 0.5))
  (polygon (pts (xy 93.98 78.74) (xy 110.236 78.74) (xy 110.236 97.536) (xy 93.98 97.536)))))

